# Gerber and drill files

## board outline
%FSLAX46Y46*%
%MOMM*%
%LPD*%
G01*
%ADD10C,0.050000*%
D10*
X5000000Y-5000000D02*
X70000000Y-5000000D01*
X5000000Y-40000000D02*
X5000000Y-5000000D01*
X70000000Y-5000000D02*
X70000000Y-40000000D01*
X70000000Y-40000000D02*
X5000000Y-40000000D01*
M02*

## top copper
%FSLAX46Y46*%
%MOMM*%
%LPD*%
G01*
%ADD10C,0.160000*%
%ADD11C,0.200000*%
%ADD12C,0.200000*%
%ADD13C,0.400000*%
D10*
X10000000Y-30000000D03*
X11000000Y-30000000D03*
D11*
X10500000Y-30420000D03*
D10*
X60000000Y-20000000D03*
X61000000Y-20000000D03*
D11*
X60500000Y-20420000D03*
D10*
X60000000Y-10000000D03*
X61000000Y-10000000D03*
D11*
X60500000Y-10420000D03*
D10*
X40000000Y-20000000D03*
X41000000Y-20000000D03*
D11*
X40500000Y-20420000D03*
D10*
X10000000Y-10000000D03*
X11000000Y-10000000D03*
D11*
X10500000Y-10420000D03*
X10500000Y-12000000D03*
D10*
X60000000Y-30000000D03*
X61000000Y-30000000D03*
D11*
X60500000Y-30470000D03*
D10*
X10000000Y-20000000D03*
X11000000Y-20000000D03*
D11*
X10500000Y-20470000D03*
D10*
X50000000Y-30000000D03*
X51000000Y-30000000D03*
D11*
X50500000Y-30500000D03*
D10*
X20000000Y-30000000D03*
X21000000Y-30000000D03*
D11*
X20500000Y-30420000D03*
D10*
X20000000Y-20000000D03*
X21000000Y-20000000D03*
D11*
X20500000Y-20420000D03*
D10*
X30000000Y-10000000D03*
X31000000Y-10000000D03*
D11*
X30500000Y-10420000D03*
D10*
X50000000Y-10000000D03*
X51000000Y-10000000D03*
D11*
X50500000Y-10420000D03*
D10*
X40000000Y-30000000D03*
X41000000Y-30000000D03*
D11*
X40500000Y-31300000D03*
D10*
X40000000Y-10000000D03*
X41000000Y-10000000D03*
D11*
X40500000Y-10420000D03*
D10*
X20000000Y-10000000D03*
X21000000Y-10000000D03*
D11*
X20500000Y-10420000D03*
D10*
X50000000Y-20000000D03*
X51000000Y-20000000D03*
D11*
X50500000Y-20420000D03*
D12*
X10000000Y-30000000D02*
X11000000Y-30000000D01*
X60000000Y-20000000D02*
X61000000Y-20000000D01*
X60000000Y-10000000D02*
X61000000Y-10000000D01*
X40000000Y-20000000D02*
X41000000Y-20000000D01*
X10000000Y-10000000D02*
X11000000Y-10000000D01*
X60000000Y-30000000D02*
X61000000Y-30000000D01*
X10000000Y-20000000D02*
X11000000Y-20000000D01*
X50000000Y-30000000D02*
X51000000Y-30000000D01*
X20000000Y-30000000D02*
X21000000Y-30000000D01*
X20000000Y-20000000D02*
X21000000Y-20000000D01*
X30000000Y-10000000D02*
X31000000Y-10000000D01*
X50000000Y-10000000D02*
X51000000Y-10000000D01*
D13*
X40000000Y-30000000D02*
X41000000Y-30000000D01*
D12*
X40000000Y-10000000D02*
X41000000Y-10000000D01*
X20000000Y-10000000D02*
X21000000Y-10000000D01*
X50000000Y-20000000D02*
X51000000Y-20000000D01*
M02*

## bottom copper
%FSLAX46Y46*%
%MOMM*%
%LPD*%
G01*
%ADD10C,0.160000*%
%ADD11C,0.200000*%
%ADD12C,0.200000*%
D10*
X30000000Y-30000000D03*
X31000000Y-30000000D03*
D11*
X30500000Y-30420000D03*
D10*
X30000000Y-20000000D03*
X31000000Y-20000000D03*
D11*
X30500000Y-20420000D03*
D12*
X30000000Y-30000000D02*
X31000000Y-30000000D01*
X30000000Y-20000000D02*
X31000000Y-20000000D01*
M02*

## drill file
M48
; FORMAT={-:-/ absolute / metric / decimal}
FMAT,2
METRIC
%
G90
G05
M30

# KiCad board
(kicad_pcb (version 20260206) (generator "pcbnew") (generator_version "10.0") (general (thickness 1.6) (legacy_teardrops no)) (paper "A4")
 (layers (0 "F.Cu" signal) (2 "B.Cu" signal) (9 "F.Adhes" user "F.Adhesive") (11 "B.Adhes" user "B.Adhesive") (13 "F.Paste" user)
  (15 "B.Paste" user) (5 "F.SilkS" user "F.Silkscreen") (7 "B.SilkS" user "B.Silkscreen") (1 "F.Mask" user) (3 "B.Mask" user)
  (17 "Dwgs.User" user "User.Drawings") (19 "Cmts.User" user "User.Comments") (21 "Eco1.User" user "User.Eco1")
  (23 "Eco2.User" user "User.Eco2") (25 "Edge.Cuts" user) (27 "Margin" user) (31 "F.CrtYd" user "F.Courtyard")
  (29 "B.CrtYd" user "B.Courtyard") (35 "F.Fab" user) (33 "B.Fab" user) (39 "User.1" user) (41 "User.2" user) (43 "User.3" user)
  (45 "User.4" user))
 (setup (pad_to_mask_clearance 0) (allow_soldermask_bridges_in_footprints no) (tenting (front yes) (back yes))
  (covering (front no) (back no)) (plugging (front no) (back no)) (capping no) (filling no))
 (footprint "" (layer "F.Cu") (at 10 30)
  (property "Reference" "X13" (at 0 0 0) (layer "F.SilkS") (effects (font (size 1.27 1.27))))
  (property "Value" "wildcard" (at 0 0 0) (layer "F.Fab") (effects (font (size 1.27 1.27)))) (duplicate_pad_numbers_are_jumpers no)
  (pad "1" smd circle (at 0 0) (size 0.16 0.16) (layers "F.Cu") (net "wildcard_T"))
  (pad "2" smd circle (at 1 0) (size 0.16 0.16) (layers "F.Cu") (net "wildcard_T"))
  (pad "3" smd circle (at 0.5 0.42) (size 0.2 0.2) (layers "F.Cu") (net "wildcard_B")))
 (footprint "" (layer "F.Cu") (at 60 20)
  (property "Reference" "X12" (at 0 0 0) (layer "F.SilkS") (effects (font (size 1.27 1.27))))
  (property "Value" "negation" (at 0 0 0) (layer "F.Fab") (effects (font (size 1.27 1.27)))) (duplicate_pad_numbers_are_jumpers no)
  (pad "1" smd circle (at 0 0) (size 0.16 0.16) (layers "F.Cu") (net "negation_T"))
  (pad "2" smd circle (at 1 0) (size 0.16 0.16) (layers "F.Cu") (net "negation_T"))
  (pad "3" smd circle (at 0.5 0.42) (size 0.2 0.2) (layers "F.Cu") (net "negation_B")))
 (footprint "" (layer "F.Cu") (at 60 10)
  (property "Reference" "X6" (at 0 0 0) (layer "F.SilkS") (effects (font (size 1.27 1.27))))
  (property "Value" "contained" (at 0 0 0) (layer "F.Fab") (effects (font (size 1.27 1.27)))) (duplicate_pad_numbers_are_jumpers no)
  (pad "1" smd circle (at 0 0) (size 0.16 0.16) (layers "F.Cu") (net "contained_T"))
  (pad "2" smd circle (at 1 0) (size 0.16 0.16) (layers "F.Cu") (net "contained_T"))
  (pad "3" smd circle (at 0.5 0.42) (size 0.2 0.2) (layers "F.Cu") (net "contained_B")))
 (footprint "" (layer "F.Cu") (at 40 20)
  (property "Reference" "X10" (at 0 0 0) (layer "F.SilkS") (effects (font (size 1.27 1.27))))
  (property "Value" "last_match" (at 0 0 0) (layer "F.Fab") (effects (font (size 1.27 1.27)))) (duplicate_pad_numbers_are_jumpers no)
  (pad "1" smd circle (at 0 0) (size 0.16 0.16) (layers "F.Cu") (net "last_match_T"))
  (pad "2" smd circle (at 1 0) (size 0.16 0.16) (layers "F.Cu") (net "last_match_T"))
  (pad "3" smd circle (at 0.5 0.42) (size 0.2 0.2) (layers "F.Cu") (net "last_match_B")))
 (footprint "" (layer "F.Cu") (at 10 10)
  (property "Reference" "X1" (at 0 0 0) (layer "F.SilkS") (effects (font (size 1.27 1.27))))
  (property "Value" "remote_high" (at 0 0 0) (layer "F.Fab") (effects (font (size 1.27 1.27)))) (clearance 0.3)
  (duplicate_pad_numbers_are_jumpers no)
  (pad "1" smd circle (at 0 0) (size 0.16 0.16) (layers "F.Cu") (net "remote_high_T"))
  (pad "2" smd circle (at 1 0) (size 0.16 0.16) (layers "F.Cu") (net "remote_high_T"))
  (pad "3" smd circle (at 0.5 0.42) (size 0.2 0.2) (layers "F.Cu") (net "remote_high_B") (clearance 0))
  (pad "4" smd circle (at 0.5 2) (size 0.2 0.2) (layers "F.Cu") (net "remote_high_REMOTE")))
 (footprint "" (layer "F.Cu") (at 60 30)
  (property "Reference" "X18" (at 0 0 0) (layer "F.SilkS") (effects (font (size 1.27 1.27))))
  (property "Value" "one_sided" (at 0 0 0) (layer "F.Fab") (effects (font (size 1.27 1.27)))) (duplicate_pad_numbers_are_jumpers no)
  (pad "1" smd circle (at 0 0) (size 0.16 0.16) (layers "F.Cu") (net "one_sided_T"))
  (pad "2" smd circle (at 1 0) (size 0.16 0.16) (layers "F.Cu") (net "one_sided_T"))
  (pad "3" smd circle (at 0.5 0.47) (size 0.2 0.2) (layers "F.Cu") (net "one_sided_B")))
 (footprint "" (layer "F.Cu") (at 10 20)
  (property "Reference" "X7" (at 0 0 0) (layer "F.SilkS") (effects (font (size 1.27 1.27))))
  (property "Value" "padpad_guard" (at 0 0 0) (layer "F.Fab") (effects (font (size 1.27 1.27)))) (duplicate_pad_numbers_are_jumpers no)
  (pad "1" smd circle (at 0 0) (size 0.16 0.16) (layers "F.Cu") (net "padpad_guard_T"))
  (pad "2" smd circle (at 1 0) (size 0.16 0.16) (layers "F.Cu") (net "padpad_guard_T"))
  (pad "3" smd circle (at 0.5 0.47) (size 0.2 0.2) (layers "F.Cu") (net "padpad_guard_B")))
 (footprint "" (layer "F.Cu") (at 50 30)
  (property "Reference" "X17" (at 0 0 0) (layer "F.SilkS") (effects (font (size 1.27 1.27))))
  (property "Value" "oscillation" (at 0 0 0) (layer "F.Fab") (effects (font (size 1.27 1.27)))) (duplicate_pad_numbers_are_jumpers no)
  (pad "1" smd circle (at 0 0) (size 0.16 0.16) (layers "F.Cu") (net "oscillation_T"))
  (pad "2" smd circle (at 1 0) (size 0.16 0.16) (layers "F.Cu") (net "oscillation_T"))
  (pad "3" smd circle (at 0.5 0.5) (size 0.2 0.2) (layers "F.Cu") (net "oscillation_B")))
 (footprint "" (layer "F.Cu") (at 20 30)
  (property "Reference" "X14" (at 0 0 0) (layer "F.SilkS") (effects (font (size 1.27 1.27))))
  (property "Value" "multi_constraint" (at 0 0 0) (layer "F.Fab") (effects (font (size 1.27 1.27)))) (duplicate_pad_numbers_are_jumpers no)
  (pad "1" smd circle (at 0 0) (size 0.16 0.16) (layers "F.Cu") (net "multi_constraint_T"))
  (pad "2" smd circle (at 1 0) (size 0.16 0.16) (layers "F.Cu") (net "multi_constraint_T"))
  (pad "3" smd circle (at 0.5 0.42) (size 0.2 0.2) (layers "F.Cu") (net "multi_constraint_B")))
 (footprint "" (layer "F.Cu") (at 30 30)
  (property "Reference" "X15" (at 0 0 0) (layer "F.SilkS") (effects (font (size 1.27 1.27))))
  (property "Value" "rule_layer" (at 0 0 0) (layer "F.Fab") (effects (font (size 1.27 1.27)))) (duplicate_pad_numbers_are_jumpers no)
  (pad "1" smd circle (at 0 0) (size 0.16 0.16) (layers "B.Cu") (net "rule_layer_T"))
  (pad "2" smd circle (at 1 0) (size 0.16 0.16) (layers "B.Cu") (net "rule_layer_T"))
  (pad "3" smd circle (at 0.5 0.42) (size 0.2 0.2) (layers "B.Cu") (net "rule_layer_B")))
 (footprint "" (layer "F.Cu") (at 20 20)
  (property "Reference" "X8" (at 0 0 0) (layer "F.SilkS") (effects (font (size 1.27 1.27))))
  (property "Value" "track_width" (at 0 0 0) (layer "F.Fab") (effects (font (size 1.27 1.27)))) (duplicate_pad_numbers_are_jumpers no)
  (pad "1" smd circle (at 0 0) (size 0.16 0.16) (layers "F.Cu") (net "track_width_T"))
  (pad "2" smd circle (at 1 0) (size 0.16 0.16) (layers "F.Cu") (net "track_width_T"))
  (pad "3" smd circle (at 0.5 0.42) (size 0.2 0.2) (layers "F.Cu") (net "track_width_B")))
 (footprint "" (layer "F.Cu") (at 30 10)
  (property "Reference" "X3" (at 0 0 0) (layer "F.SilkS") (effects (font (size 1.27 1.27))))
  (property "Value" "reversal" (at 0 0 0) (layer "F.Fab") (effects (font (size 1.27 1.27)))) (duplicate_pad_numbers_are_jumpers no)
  (pad "1" smd circle (at 0 0) (size 0.16 0.16) (layers "F.Cu") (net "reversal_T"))
  (pad "2" smd circle (at 1 0) (size 0.16 0.16) (layers "F.Cu") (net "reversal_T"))
  (pad "3" smd circle (at 0.5 0.42) (size 0.2 0.2) (layers "F.Cu") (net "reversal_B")))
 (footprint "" (layer "F.Cu") (at 50 10)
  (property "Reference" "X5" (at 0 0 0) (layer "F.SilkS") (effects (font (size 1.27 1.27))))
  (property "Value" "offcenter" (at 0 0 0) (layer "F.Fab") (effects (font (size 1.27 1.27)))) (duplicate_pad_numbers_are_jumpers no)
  (pad "1" smd circle (at 0 0) (size 0.16 0.16) (layers "F.Cu") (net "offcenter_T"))
  (pad "2" smd circle (at 1 0) (size 0.16 0.16) (layers "F.Cu") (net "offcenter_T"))
  (pad "3" smd circle (at 0.5 0.42) (size 0.2 0.2) (layers "F.Cu") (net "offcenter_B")))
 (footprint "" (layer "F.Cu") (at 40 30)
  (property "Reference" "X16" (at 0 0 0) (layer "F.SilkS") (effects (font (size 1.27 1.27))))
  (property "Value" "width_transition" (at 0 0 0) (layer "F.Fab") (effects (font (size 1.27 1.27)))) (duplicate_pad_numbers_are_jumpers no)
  (pad "1" smd circle (at 0 0) (size 0.16 0.16) (layers "F.Cu") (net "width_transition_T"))
  (pad "2" smd circle (at 1 0) (size 0.16 0.16) (layers "F.Cu") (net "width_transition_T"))
  (pad "3" smd circle (at 0.5 1.3) (size 0.2 0.2) (layers "F.Cu") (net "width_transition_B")))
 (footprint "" (layer "F.Cu") (at 30 20)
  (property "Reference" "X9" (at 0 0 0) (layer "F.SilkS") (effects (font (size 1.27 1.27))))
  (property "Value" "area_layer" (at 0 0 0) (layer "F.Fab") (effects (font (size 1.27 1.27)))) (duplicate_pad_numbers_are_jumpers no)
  (pad "1" smd circle (at 0 0) (size 0.16 0.16) (layers "B.Cu") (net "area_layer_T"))
  (pad "2" smd circle (at 1 0) (size 0.16 0.16) (layers "B.Cu") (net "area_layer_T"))
  (pad "3" smd circle (at 0.5 0.42) (size 0.2 0.2) (layers "B.Cu") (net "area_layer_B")))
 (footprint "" (layer "F.Cu") (at 40 10)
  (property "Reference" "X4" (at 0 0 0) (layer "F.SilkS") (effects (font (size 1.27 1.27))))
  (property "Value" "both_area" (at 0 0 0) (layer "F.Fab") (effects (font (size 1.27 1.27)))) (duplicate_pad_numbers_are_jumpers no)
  (pad "1" smd circle (at 0 0) (size 0.16 0.16) (layers "F.Cu") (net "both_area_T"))
  (pad "2" smd circle (at 1 0) (size 0.16 0.16) (layers "F.Cu") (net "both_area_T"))
  (pad "3" smd circle (at 0.5 0.42) (size 0.2 0.2) (layers "F.Cu") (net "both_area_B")))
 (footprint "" (layer "F.Cu") (at 20 10)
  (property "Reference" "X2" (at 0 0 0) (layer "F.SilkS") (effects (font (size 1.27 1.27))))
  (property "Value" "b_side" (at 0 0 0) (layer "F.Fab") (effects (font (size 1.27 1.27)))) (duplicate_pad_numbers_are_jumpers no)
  (pad "1" smd circle (at 0 0) (size 0.16 0.16) (layers "F.Cu") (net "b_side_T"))
  (pad "2" smd circle (at 1 0) (size 0.16 0.16) (layers "F.Cu") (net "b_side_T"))
  (pad "3" smd circle (at 0.5 0.42) (size 0.2 0.2) (layers "F.Cu") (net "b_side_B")))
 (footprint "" (layer "F.Cu") (at 50 20)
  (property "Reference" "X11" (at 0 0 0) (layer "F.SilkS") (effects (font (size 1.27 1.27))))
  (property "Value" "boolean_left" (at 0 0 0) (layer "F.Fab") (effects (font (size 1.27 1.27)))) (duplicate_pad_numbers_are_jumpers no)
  (pad "1" smd circle (at 0 0) (size 0.16 0.16) (layers "F.Cu") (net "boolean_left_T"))
  (pad "2" smd circle (at 1 0) (size 0.16 0.16) (layers "F.Cu") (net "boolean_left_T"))
  (pad "3" smd circle (at 0.5 0.42) (size 0.2 0.2) (layers "F.Cu") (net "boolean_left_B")))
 (gr_line (start 5 5) (end 70 5) (stroke (width 0.05) (type default)) (layer "Edge.Cuts"))
 (gr_line (start 5 40) (end 5 5) (stroke (width 0.05) (type default)) (layer "Edge.Cuts"))
 (gr_line (start 70 5) (end 70 40) (stroke (width 0.05) (type default)) (layer "Edge.Cuts"))
 (gr_line (start 70 40) (end 5 40) (stroke (width 0.05) (type default)) (layer "Edge.Cuts"))
 (segment (start 10 30) (end 11 30) (width 0.2) (layer "F.Cu") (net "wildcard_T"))
 (segment (start 60 20) (end 61 20) (width 0.2) (layer "F.Cu") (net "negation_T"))
 (segment (start 60 10) (end 61 10) (width 0.2) (layer "F.Cu") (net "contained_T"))
 (segment (start 40 20) (end 41 20) (width 0.2) (layer "F.Cu") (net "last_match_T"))
 (segment (start 10 10) (end 11 10) (width 0.2) (layer "F.Cu") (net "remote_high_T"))
 (segment (start 60 30) (end 61 30) (width 0.2) (layer "F.Cu") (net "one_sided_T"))
 (segment (start 10 20) (end 11 20) (width 0.2) (layer "F.Cu") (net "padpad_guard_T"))
 (segment (start 50 30) (end 51 30) (width 0.2) (layer "F.Cu") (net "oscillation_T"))
 (segment (start 20 30) (end 21 30) (width 0.2) (layer "F.Cu") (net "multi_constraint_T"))
 (segment (start 30 30) (end 31 30) (width 0.2) (layer "B.Cu") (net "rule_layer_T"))
 (segment (start 20 20) (end 21 20) (width 0.2) (layer "F.Cu") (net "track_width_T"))
 (segment (start 30 10) (end 31 10) (width 0.2) (layer "F.Cu") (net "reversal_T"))
 (segment (start 50 10) (end 51 10) (width 0.2) (layer "F.Cu") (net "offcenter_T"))
 (segment (start 40 30) (end 41 30) (width 0.4) (layer "F.Cu") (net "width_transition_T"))
 (segment (start 30 20) (end 31 20) (width 0.2) (layer "B.Cu") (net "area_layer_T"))
 (segment (start 40 10) (end 41 10) (width 0.2) (layer "F.Cu") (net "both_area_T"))
 (segment (start 20 10) (end 21 10) (width 0.2) (layer "F.Cu") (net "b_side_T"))
 (segment (start 50 20) (end 51 20) (width 0.2) (layer "F.Cu") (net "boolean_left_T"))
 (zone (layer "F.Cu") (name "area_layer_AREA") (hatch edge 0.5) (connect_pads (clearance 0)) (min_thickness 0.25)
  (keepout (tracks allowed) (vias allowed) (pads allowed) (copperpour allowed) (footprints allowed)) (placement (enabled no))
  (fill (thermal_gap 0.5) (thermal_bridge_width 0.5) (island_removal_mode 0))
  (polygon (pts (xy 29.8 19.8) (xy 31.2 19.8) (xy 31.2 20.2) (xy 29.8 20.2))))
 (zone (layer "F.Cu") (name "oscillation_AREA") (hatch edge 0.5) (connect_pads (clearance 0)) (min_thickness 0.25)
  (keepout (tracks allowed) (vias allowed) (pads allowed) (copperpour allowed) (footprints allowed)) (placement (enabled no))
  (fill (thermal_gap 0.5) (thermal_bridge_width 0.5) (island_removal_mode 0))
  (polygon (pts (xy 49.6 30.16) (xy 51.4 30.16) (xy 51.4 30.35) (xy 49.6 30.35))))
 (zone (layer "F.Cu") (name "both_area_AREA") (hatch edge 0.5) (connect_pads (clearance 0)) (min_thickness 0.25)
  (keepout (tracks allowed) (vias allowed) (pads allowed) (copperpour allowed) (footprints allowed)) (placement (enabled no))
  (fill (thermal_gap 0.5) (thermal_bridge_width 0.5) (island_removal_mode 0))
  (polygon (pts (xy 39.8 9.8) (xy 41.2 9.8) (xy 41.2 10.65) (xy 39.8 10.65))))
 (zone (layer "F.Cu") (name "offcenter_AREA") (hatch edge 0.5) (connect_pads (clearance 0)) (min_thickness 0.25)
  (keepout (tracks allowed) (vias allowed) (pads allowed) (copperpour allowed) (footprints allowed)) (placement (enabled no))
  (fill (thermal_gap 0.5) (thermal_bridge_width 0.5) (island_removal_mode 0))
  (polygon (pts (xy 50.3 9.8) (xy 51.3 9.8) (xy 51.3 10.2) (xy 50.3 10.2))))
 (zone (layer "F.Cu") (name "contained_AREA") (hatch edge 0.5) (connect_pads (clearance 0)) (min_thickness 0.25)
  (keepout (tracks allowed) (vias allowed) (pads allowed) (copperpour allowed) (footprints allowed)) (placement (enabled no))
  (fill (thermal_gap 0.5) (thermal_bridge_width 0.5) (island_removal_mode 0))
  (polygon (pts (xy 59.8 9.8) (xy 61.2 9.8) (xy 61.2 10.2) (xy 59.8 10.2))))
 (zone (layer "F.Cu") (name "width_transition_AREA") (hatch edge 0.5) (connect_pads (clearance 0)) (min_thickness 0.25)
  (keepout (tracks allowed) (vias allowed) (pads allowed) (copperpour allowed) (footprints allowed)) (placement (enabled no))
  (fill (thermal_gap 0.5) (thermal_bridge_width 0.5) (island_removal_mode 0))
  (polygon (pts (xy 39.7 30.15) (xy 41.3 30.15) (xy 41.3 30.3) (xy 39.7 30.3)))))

